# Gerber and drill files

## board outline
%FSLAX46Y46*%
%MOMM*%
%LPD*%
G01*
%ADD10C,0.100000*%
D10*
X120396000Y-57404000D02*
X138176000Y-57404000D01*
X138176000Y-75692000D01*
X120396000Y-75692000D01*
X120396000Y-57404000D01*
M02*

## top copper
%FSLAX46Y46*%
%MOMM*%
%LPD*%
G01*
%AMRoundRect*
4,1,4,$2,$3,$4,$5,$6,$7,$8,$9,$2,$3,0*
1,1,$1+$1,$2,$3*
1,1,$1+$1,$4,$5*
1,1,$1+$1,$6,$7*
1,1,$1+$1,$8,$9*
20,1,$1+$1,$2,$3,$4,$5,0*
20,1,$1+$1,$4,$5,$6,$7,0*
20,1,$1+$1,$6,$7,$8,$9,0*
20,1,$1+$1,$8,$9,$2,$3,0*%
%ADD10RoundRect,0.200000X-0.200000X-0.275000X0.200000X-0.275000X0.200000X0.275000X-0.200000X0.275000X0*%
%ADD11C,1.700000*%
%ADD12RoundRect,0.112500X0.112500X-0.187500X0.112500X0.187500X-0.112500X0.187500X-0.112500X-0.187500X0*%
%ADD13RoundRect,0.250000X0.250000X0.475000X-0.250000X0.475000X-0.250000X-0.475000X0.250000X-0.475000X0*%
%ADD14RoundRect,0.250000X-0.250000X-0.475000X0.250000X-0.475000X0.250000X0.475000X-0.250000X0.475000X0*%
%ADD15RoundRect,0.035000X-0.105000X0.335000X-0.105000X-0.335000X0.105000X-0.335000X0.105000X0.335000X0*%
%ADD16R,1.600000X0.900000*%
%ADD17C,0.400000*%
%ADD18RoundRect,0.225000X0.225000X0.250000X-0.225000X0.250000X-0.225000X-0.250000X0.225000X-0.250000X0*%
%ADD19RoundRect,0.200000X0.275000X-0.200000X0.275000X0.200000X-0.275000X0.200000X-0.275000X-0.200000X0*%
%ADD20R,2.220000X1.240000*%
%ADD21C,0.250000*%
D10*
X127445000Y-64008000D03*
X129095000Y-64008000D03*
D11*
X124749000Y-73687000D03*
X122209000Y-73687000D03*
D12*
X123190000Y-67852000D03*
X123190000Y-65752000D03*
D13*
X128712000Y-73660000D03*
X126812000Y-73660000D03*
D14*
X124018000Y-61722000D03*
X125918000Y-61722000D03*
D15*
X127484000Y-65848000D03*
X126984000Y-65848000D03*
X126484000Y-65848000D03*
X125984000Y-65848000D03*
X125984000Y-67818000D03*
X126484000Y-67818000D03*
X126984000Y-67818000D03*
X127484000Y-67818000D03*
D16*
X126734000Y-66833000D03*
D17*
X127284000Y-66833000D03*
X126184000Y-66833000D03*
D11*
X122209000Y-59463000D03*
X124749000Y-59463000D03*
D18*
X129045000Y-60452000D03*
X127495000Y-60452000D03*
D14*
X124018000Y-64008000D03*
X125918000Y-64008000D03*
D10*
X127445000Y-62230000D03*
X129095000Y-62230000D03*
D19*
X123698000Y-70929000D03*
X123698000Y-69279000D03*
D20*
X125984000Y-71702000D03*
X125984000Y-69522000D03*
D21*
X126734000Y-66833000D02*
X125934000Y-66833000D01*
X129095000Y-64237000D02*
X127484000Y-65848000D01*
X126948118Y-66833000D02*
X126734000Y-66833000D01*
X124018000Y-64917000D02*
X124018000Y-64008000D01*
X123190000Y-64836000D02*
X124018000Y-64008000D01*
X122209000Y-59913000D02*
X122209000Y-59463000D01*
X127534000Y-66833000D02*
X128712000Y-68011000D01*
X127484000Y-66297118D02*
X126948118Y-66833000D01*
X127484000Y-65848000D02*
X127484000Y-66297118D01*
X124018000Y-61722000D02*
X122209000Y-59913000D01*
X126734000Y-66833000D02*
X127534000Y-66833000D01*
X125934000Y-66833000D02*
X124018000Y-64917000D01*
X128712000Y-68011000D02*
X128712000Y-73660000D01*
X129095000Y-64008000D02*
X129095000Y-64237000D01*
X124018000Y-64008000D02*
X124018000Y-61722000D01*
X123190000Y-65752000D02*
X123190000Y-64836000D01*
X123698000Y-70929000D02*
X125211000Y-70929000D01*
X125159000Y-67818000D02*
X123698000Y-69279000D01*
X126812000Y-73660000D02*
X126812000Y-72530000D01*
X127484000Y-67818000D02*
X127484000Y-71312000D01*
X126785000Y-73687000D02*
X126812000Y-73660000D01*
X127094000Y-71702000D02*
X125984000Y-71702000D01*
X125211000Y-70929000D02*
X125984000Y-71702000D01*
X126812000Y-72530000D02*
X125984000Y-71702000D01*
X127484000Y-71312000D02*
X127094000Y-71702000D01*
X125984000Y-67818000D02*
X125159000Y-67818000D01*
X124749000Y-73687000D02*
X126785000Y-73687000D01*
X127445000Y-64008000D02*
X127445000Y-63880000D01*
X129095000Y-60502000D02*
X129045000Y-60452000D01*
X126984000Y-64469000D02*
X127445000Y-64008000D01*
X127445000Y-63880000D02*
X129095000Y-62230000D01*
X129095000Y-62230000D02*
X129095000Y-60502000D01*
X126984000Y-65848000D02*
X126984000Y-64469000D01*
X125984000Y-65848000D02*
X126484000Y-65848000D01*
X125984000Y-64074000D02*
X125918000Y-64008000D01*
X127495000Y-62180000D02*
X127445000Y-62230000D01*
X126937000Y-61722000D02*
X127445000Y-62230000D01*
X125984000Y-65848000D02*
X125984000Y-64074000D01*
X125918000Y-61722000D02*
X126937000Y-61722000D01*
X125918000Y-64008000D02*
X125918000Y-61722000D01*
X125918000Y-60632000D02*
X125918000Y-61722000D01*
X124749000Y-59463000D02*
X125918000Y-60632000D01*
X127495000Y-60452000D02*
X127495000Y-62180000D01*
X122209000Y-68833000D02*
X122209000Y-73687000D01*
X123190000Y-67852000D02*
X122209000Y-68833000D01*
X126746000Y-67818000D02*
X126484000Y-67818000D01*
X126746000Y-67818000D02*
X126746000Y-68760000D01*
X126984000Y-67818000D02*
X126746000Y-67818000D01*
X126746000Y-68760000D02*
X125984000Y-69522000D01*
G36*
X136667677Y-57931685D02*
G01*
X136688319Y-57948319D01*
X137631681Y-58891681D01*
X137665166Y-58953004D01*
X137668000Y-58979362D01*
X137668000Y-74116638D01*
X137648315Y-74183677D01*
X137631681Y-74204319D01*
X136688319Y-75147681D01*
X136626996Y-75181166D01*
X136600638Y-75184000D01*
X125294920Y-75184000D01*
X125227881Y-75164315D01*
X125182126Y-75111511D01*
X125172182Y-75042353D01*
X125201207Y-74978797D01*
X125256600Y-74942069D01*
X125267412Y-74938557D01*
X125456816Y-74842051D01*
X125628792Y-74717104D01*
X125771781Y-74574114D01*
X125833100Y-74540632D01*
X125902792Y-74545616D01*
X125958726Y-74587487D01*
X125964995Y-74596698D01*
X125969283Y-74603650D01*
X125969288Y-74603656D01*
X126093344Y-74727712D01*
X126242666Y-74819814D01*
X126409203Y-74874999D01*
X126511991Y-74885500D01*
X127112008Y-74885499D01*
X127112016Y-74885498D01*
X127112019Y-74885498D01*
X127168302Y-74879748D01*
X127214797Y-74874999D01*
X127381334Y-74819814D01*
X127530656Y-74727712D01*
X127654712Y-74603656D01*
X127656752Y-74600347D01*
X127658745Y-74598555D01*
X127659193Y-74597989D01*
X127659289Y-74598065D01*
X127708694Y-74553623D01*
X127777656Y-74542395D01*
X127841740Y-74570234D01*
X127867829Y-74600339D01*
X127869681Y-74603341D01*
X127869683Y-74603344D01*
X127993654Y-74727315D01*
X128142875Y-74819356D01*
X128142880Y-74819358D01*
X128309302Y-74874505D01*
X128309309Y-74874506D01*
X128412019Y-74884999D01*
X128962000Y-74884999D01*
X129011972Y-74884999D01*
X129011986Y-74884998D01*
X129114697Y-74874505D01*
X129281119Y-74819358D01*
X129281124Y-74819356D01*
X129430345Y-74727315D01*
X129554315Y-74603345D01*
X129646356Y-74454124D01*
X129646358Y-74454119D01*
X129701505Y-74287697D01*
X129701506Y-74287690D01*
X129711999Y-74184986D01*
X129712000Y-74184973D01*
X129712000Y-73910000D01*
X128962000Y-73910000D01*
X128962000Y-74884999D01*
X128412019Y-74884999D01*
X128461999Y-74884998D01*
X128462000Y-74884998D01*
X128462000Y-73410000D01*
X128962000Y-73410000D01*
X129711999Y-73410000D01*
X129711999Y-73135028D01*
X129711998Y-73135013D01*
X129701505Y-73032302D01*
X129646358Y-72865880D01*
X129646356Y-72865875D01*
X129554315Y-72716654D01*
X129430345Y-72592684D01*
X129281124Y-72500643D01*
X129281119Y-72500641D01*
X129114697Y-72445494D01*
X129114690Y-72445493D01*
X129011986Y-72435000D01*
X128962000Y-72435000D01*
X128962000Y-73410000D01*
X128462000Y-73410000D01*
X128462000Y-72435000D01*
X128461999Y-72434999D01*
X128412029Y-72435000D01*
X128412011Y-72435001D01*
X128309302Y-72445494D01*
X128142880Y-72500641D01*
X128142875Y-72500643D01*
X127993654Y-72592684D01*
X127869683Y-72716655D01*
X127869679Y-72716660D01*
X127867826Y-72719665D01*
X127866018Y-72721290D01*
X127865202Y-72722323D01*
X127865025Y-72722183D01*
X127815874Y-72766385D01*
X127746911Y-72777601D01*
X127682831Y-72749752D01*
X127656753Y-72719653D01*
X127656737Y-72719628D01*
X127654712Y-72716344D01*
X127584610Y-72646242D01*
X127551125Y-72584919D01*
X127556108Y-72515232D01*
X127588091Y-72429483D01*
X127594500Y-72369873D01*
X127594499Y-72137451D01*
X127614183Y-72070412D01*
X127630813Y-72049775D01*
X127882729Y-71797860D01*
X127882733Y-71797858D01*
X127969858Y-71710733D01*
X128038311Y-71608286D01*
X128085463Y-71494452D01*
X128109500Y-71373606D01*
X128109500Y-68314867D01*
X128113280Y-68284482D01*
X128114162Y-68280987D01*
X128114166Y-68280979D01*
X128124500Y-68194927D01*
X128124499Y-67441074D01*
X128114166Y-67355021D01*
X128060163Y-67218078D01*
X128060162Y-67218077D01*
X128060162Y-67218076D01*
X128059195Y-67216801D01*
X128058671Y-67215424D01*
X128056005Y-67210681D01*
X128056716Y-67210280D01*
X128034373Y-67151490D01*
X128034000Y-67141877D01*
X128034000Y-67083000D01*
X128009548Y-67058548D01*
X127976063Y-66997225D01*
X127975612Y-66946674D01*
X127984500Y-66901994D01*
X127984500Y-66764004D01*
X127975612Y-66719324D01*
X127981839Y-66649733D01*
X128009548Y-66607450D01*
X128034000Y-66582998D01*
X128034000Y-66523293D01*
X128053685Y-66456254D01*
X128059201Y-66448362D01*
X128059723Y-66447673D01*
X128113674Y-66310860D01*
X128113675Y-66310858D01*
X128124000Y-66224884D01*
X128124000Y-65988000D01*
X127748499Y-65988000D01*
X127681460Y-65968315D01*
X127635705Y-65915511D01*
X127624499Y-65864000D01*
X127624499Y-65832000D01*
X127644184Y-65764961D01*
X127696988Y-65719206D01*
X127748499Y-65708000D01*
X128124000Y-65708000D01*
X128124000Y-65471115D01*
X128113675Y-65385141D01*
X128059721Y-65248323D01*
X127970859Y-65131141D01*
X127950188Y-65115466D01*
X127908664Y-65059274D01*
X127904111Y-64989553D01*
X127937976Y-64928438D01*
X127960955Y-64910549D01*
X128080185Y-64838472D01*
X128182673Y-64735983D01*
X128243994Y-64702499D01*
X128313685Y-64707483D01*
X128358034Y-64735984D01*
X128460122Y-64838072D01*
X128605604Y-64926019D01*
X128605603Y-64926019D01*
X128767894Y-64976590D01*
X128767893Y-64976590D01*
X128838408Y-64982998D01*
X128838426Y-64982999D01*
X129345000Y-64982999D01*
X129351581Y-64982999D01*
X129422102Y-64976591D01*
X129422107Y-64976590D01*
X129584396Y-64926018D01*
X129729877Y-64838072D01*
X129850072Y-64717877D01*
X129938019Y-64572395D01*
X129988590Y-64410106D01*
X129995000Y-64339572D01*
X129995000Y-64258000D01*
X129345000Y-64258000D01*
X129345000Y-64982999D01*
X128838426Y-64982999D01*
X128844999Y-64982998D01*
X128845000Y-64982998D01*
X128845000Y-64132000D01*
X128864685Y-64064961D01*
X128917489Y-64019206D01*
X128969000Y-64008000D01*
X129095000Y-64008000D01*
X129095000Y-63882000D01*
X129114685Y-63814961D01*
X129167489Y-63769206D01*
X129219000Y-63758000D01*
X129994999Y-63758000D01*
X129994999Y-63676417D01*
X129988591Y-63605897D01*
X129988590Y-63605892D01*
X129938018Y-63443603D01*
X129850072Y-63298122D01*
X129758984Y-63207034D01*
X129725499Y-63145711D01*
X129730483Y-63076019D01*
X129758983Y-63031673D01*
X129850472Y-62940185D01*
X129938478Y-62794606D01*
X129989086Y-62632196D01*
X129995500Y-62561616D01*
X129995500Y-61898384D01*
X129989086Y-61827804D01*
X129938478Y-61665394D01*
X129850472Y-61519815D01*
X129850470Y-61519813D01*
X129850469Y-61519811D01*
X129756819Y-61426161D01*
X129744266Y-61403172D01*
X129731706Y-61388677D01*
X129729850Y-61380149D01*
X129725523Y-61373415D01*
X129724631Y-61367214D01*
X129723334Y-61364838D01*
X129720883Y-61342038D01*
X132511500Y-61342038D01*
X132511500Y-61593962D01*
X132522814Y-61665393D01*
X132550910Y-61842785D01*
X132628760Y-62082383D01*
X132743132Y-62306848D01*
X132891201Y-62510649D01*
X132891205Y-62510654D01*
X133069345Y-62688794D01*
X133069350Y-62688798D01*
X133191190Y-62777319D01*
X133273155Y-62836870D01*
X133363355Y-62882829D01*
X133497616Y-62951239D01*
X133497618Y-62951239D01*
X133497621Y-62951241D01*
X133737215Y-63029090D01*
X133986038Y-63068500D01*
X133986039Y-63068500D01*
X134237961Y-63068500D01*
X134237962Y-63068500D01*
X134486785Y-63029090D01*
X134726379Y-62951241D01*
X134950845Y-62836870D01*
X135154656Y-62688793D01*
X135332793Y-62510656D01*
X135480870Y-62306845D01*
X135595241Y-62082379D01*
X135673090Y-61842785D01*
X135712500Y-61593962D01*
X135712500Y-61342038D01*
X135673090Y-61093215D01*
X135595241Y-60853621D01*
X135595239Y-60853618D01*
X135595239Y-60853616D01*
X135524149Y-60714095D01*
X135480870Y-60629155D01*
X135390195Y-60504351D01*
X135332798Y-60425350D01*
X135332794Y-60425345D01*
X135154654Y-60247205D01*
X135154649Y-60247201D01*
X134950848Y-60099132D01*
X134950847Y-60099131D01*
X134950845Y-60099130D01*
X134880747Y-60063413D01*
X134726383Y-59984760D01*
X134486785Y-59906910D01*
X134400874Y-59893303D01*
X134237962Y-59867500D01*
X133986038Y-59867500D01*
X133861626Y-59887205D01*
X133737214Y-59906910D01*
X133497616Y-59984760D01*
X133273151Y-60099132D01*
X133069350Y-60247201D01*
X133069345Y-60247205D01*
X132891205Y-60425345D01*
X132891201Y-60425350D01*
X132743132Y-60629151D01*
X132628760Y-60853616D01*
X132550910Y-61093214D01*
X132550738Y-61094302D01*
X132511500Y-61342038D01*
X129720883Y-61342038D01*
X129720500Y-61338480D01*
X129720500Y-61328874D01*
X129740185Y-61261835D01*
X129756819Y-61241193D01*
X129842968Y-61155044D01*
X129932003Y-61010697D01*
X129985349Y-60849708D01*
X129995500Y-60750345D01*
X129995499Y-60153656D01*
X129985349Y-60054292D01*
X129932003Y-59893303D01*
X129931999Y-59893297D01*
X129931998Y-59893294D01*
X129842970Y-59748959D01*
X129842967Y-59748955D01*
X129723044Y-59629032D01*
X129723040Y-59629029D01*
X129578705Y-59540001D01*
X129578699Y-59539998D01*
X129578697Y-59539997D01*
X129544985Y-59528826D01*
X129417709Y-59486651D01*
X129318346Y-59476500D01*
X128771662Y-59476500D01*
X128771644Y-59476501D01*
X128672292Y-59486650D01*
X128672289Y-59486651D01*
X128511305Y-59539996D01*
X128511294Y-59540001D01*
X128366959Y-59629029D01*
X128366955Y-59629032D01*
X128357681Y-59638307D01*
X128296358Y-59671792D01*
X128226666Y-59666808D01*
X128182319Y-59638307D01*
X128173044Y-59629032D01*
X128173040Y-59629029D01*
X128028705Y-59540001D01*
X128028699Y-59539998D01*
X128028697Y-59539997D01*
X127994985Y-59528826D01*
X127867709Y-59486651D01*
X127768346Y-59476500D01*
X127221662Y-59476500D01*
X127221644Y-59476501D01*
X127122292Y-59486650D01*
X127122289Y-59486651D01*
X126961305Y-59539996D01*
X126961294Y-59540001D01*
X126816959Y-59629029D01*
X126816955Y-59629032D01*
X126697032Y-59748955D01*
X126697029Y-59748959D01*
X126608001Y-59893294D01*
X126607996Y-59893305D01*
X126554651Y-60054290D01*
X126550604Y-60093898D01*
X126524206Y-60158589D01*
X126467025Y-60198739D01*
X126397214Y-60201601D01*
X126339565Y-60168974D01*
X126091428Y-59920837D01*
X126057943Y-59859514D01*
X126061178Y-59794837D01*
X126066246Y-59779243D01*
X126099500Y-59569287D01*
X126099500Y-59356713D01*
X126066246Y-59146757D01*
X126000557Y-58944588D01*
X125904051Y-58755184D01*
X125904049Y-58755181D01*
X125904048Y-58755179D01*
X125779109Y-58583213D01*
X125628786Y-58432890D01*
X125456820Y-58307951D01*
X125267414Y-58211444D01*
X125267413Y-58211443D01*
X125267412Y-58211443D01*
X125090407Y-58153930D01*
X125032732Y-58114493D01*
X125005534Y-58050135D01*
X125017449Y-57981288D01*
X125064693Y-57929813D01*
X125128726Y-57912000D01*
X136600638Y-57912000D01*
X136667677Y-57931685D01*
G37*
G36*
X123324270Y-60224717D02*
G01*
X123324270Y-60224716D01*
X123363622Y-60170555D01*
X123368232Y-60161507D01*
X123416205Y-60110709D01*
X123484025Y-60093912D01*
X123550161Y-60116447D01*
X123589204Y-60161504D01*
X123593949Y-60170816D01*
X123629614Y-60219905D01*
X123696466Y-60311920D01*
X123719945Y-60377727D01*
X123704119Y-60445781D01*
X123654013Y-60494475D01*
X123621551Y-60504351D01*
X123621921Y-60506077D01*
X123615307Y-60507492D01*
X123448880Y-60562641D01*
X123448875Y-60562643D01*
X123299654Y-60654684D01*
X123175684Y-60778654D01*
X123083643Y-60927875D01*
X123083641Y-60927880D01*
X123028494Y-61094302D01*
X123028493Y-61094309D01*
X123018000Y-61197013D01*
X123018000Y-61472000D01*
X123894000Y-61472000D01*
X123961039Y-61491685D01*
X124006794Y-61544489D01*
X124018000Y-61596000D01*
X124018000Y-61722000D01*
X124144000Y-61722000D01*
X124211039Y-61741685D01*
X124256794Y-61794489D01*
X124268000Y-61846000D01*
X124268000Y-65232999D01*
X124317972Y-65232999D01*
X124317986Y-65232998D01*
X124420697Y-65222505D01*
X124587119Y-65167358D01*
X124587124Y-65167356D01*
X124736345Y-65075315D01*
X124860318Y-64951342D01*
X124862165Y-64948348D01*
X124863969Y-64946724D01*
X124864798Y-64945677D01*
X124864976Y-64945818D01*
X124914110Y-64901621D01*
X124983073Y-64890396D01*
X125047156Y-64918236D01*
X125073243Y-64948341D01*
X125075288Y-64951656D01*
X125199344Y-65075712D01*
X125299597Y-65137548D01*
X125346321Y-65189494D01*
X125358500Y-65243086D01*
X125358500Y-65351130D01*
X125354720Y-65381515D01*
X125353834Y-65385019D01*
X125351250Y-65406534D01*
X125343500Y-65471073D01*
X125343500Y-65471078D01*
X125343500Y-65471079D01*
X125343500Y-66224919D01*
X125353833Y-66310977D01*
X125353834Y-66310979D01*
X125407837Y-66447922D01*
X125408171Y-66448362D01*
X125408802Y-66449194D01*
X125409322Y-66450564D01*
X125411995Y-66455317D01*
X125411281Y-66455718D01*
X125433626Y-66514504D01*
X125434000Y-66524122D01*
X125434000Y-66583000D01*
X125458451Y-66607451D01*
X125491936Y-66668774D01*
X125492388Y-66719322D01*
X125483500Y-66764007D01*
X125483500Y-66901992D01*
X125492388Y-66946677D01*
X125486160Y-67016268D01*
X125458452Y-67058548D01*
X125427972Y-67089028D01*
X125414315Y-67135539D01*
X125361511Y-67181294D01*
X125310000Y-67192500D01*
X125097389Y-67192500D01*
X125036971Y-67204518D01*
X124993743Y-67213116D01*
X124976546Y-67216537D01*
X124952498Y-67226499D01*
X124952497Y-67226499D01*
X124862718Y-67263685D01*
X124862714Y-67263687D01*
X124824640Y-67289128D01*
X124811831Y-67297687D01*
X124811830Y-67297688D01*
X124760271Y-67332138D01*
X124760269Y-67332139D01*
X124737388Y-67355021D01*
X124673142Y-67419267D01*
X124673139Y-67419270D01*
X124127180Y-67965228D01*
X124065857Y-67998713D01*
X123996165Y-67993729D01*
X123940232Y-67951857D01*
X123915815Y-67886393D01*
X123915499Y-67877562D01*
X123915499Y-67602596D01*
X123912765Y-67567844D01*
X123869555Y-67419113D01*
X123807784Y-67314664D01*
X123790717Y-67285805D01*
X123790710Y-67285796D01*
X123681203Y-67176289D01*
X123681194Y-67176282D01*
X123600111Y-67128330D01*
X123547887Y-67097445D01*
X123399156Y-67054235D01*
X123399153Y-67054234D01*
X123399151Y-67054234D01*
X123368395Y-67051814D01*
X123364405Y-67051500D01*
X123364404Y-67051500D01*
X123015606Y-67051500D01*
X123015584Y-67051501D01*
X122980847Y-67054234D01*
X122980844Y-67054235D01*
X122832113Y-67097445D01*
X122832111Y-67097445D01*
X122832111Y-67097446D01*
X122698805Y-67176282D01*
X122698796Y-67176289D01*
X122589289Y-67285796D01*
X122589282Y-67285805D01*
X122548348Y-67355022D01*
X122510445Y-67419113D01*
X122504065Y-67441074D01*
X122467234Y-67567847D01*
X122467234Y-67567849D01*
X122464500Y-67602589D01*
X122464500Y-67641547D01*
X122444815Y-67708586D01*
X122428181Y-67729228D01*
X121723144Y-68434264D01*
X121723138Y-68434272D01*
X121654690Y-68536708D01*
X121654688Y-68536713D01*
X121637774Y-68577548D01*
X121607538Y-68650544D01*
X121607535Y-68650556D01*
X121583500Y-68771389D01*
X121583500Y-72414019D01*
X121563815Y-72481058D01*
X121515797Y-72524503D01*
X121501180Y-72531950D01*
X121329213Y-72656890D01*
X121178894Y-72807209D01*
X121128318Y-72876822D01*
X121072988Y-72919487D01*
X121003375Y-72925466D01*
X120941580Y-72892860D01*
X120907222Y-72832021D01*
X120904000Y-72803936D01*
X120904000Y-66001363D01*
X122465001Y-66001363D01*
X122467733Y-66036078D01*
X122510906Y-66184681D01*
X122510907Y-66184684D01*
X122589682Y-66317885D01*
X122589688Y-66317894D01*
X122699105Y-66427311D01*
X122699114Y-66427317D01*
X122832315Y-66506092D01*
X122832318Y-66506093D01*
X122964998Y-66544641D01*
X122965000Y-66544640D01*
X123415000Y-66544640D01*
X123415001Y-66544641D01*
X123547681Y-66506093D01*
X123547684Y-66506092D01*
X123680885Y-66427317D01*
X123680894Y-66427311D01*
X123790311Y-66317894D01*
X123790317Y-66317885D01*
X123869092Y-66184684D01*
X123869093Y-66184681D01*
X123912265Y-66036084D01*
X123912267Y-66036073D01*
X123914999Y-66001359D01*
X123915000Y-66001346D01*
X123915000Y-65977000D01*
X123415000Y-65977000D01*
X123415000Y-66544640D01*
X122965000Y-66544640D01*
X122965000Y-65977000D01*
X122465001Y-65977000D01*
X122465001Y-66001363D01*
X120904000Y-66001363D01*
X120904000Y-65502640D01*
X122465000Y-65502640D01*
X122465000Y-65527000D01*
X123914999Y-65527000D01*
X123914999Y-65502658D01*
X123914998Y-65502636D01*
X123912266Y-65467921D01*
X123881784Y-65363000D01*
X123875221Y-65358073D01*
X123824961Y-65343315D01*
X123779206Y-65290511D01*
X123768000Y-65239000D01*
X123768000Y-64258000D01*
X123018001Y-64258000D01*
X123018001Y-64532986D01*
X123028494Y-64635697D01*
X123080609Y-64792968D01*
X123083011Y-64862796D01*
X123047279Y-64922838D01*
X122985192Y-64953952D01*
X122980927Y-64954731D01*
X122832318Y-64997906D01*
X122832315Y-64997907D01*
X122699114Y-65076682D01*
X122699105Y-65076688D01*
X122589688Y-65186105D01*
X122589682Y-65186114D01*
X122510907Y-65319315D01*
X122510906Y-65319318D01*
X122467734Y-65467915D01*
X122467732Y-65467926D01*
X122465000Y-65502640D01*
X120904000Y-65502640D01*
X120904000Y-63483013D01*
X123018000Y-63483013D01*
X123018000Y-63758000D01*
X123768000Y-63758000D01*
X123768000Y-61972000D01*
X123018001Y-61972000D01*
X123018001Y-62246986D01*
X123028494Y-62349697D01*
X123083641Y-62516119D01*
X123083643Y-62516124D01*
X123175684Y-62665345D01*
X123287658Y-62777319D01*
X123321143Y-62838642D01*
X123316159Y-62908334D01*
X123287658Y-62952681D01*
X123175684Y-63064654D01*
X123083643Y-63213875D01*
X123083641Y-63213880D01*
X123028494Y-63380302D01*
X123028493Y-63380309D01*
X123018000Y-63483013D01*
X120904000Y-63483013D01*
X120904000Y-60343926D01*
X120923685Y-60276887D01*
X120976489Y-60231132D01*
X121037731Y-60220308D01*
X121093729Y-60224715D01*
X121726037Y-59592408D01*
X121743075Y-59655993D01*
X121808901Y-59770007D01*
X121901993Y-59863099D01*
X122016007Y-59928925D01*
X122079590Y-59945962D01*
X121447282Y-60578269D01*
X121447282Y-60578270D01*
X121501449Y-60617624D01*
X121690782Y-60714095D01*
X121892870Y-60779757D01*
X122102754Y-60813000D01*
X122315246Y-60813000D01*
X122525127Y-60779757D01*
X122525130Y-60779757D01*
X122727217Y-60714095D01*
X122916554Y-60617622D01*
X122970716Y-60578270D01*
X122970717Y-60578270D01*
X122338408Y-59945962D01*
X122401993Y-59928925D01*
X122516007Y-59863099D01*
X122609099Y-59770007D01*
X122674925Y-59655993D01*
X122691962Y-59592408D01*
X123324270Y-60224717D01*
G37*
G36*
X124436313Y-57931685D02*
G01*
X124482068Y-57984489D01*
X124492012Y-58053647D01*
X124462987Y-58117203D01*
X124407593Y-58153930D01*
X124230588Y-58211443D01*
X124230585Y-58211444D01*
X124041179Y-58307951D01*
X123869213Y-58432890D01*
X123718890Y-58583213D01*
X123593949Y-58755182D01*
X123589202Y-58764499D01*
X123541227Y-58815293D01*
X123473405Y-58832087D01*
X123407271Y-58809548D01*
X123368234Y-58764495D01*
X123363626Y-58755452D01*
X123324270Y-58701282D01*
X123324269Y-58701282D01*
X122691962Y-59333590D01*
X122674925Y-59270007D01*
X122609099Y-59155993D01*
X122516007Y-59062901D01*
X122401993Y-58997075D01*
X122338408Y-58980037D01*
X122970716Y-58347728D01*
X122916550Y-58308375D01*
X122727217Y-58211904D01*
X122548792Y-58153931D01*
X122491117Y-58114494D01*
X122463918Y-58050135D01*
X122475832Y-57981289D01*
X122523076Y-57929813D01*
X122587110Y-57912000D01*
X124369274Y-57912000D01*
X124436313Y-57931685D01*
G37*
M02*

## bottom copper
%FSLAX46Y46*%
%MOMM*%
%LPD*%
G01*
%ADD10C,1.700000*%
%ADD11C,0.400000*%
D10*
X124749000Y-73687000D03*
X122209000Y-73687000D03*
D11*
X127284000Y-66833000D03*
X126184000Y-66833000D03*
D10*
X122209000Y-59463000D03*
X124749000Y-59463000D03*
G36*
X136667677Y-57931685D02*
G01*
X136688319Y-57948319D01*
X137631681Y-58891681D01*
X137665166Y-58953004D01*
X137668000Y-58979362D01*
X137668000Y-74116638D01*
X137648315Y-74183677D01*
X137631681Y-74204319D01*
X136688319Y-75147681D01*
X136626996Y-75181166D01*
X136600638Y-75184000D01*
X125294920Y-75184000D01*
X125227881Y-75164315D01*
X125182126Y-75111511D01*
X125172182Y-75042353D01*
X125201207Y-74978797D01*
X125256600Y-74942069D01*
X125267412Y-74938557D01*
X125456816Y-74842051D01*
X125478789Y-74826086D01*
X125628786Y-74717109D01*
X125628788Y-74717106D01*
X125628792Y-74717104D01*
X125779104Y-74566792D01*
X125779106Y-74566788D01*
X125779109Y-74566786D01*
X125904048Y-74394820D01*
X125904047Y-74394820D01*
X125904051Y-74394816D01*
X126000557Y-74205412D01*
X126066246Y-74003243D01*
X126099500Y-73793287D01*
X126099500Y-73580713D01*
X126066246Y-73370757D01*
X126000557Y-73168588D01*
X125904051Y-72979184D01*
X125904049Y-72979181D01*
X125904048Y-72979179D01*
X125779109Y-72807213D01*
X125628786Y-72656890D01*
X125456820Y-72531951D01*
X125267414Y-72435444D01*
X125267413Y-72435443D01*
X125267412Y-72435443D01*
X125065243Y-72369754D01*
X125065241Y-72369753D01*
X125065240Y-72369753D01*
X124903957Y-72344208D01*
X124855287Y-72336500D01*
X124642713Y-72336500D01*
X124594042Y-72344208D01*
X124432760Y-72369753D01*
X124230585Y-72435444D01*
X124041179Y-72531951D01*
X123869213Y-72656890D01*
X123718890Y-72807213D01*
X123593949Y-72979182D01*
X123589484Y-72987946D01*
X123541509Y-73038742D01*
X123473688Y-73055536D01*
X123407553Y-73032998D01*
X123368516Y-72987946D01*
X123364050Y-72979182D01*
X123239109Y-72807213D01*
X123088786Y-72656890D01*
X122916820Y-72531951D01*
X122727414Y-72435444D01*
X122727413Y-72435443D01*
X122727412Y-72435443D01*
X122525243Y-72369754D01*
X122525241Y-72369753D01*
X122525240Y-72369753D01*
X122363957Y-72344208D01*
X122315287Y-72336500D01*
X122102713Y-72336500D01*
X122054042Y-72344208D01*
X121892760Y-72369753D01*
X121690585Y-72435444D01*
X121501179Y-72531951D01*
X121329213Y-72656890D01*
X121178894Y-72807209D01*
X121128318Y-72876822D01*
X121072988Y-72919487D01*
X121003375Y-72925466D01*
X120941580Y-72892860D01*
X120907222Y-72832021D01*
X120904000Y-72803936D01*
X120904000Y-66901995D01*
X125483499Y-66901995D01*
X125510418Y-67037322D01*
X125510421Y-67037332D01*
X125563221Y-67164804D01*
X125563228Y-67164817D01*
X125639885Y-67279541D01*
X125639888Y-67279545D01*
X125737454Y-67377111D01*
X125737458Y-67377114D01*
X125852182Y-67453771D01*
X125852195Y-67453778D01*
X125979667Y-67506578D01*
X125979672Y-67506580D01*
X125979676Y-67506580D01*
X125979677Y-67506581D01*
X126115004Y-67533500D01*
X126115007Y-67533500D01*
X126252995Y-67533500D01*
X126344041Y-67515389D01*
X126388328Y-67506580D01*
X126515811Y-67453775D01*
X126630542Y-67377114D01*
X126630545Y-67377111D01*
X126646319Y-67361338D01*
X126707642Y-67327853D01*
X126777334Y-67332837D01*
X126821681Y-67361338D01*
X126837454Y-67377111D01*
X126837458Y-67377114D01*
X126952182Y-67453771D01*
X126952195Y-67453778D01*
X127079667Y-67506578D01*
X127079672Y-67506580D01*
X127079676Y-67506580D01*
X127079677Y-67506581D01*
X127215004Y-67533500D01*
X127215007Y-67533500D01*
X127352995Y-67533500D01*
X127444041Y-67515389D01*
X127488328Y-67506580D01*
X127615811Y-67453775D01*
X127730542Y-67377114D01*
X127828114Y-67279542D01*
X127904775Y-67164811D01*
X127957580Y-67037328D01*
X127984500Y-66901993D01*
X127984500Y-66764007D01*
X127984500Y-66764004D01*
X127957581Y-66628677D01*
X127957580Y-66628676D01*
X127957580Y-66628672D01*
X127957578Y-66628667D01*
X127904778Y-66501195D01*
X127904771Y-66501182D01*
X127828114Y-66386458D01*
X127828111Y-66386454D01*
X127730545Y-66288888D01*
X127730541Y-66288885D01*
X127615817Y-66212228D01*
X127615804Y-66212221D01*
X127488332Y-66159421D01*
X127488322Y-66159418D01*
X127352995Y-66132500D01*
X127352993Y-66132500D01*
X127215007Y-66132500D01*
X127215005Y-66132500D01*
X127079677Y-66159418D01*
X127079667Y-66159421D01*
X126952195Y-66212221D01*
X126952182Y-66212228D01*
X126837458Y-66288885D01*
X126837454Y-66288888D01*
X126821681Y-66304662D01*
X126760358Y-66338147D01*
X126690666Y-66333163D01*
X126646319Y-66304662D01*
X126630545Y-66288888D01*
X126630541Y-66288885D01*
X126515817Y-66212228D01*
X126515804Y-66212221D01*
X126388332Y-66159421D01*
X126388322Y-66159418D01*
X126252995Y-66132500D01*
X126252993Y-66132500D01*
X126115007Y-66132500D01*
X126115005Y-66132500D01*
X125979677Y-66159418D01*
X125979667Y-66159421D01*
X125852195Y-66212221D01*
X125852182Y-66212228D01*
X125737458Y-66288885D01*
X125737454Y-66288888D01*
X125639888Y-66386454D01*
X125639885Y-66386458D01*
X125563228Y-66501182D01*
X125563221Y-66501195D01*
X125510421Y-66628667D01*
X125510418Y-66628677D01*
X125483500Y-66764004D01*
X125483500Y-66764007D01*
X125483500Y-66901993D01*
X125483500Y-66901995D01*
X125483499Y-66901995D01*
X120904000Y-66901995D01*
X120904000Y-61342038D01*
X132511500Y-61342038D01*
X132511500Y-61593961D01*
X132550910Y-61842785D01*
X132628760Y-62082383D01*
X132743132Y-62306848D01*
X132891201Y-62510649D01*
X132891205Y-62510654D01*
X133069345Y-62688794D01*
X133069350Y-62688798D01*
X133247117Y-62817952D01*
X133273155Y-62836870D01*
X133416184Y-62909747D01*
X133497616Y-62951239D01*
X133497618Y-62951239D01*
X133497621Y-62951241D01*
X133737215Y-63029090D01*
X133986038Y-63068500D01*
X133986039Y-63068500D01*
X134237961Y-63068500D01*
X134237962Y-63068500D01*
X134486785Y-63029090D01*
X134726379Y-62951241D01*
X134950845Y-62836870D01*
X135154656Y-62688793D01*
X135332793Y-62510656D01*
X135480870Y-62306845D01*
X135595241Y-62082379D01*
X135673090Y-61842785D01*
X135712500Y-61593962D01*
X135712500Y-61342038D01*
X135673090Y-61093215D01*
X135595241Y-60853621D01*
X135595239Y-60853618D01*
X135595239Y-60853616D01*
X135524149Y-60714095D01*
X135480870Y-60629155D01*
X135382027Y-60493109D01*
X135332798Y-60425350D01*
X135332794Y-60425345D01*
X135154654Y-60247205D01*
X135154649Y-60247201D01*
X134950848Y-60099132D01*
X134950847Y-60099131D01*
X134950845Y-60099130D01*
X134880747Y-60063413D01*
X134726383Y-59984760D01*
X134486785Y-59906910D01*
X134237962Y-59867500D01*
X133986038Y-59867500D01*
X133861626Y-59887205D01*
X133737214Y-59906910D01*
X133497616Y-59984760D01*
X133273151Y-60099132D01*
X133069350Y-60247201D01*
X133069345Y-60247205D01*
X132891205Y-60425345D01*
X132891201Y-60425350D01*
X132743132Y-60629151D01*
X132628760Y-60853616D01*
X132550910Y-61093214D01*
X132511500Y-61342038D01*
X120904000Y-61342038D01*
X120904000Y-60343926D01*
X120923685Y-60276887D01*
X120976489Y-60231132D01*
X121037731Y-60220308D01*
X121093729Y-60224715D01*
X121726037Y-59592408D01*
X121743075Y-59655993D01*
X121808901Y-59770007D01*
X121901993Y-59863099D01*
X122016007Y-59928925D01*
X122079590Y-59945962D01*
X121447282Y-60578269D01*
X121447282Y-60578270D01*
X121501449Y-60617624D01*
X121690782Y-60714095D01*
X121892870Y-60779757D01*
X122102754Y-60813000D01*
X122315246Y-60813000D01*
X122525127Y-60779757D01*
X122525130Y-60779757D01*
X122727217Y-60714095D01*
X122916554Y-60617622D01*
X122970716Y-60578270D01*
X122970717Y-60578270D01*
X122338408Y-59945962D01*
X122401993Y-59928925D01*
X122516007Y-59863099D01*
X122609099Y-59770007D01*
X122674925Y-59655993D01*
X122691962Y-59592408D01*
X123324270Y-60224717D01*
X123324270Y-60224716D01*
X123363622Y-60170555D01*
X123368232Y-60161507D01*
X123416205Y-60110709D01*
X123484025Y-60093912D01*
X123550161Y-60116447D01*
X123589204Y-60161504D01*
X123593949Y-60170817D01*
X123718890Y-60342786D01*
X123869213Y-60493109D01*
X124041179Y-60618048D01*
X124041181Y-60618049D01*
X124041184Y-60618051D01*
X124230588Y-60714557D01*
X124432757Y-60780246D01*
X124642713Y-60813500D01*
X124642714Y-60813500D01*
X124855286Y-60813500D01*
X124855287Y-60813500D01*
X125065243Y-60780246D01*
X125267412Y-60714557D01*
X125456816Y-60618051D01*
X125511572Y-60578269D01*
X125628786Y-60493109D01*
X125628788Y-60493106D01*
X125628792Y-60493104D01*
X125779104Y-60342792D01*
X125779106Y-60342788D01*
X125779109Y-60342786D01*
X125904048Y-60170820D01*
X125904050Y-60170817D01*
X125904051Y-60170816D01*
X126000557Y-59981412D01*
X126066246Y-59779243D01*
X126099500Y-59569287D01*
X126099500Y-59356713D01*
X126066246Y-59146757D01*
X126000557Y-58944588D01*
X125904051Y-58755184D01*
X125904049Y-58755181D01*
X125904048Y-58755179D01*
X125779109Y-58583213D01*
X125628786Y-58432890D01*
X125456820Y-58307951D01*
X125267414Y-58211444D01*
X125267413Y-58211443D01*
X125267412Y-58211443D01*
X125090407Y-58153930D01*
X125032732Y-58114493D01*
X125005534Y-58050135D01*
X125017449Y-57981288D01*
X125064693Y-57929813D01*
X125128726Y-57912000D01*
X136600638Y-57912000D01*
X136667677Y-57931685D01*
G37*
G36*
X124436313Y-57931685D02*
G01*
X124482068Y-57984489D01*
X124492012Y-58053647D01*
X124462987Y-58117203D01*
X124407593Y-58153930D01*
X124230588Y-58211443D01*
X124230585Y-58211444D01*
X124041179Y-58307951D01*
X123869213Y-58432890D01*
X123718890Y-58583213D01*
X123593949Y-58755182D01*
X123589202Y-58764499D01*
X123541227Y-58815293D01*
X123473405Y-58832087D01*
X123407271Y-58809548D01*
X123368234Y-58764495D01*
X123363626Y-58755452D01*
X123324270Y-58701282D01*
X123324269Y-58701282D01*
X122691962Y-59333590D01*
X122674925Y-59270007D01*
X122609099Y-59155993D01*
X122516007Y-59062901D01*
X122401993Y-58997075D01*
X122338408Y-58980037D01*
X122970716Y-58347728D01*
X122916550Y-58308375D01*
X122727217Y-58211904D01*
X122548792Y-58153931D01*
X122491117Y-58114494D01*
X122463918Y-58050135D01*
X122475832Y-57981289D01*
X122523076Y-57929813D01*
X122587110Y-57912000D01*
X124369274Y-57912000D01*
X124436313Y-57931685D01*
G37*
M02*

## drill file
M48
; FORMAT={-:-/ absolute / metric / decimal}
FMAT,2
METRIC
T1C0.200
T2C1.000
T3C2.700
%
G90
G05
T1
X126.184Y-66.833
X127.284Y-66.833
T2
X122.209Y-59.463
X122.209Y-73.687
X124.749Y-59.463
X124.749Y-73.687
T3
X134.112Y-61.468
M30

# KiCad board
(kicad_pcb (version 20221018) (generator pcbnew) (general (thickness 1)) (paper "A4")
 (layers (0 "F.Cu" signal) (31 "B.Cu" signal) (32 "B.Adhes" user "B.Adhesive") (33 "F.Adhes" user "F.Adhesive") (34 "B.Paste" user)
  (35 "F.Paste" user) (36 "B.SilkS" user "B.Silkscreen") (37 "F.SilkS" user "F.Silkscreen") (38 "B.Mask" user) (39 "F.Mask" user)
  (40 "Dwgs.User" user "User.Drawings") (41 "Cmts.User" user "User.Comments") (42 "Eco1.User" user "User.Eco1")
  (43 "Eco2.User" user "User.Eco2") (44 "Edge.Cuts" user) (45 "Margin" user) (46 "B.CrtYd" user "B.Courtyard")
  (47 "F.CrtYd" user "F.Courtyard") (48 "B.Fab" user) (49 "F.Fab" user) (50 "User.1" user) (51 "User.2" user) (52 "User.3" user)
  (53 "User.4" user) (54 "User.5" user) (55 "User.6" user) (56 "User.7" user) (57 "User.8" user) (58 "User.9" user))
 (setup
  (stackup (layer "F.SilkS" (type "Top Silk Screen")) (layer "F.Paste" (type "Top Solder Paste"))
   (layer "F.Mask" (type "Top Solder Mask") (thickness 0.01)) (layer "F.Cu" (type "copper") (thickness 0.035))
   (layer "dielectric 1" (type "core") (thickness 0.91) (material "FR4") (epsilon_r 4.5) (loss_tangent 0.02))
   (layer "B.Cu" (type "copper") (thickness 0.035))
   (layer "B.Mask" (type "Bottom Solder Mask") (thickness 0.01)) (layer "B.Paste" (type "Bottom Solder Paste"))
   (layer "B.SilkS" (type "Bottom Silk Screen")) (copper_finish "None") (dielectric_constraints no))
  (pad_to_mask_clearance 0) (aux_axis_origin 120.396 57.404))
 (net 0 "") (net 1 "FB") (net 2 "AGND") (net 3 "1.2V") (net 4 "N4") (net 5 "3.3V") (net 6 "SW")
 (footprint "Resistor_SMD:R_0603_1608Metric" (layer "F.Cu") (at 128.27 64.008)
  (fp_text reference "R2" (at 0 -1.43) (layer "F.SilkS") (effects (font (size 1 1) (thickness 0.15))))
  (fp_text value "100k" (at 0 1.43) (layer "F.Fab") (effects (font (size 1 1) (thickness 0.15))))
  (pad "1" smd roundrect (at -0.825 0) (size 0.8 0.95) (layers "F.Cu" "F.Paste" "F.Mask") (roundrect_rratio 0.25) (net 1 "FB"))
  (pad "2" smd roundrect (at 0.825 0) (size 0.8 0.95) (layers "F.Cu" "F.Paste" "F.Mask") (roundrect_rratio 0.25) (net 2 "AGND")))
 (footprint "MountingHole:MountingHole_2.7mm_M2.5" (layer "F.Cu") (at 134.112 61.468)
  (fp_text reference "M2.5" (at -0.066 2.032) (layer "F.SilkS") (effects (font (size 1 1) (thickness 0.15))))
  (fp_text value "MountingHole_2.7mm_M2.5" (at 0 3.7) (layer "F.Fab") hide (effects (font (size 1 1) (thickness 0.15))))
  (pad "" np_thru_hole circle (at 0 0) (size 2.7 2.7) (drill 2.7) (layers "F&B.Cu" "*.Mask")))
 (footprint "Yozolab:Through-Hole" (layer "F.Cu") (at 124.749 73.687 180)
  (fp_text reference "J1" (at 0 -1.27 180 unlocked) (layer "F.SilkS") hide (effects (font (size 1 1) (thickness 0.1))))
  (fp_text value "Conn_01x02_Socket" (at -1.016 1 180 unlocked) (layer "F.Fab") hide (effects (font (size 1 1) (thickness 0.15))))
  (pad "1" thru_hole circle (at 0 0 180) (size 1.7 1.7) (drill oval 1) (layers "*.Cu" "*.Mask") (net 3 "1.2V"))
  (pad "2" thru_hole circle (at 2.54 0 180) (size 1.7 1.7) (drill oval 1) (layers "*.Cu" "*.Mask") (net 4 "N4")))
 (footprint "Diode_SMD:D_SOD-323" (layer "F.Cu") (at 123.19 66.802 90)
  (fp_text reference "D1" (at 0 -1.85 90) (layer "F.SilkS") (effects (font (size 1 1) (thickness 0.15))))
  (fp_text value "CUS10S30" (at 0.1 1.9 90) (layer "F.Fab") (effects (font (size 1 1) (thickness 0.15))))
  (pad "1" smd roundrect (at -1.05 0 90) (size 0.6 0.45) (layers "F.Cu" "F.Paste" "F.Mask") (roundrect_rratio 0.25) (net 4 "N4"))
  (pad "2" smd roundrect (at 1.05 0 90) (size 0.6 0.45) (layers "F.Cu" "F.Paste" "F.Mask") (roundrect_rratio 0.25) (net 2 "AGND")))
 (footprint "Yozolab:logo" (layer "F.Cu") (at 136.144 70.612 90)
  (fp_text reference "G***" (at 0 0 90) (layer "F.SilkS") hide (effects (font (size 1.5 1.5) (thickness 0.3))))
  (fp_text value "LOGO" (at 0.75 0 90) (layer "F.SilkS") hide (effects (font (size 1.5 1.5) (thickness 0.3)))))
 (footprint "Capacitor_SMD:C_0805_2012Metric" (layer "F.Cu") (at 127.762 73.66 180)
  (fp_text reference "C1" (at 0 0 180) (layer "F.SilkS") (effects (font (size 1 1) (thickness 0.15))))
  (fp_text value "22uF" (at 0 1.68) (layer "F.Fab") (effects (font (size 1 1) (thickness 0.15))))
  (pad "1" smd roundrect (at -0.95 0 180) (size 1 1.45) (layers "F.Cu" "F.Paste" "F.Mask") (roundrect_rratio 0.25) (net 2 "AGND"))
  (pad "2" smd roundrect (at 0.95 0 180) (size 1 1.45) (layers "F.Cu" "F.Paste" "F.Mask") (roundrect_rratio 0.25) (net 3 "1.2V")))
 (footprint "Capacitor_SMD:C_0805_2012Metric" (layer "F.Cu") (at 124.968 61.722)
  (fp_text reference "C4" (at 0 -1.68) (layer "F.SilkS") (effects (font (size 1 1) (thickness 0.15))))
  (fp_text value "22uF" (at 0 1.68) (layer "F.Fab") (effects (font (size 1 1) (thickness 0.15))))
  (pad "1" smd roundrect (at -0.95 0) (size 1 1.45) (layers "F.Cu" "F.Paste" "F.Mask") (roundrect_rratio 0.25) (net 2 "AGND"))
  (pad "2" smd roundrect (at 0.95 0) (size 1 1.45) (layers "F.Cu" "F.Paste" "F.Mask") (roundrect_rratio 0.25) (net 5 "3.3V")))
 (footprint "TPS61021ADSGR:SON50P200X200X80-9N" (layer "F.Cu") (at 126.734 66.833 -90)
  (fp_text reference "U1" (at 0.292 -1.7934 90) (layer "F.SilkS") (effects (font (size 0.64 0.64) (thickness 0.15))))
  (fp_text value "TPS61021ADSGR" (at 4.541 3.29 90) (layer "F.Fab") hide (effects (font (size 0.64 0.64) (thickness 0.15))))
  (pad "1" smd roundrect (at -0.985 -0.75 270) (size 0.74 0.28) (layers "F.Cu" "F.Paste" "F.Mask") (roundrect_rratio 0.125) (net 2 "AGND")
   (solder_mask_margin 0.102))
  (pad "2" smd roundrect (at -0.985 -0.25 270) (size 0.74 0.28) (layers "F.Cu" "F.Paste" "F.Mask") (roundrect_rratio 0.125) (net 1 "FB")
   (solder_mask_margin 0.102))
  (pad "3" smd roundrect (at -0.985 0.25 270) (size 0.74 0.28) (layers "F.Cu" "F.Paste" "F.Mask") (roundrect_rratio 0.125) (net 5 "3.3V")
   (solder_mask_margin 0.102))
  (pad "4" smd roundrect (at -0.985 0.75 270) (size 0.74 0.28) (layers "F.Cu" "F.Paste" "F.Mask") (roundrect_rratio 0.125) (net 5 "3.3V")
   (solder_mask_margin 0.102))
  (pad "5" smd roundrect (at 0.985 0.75 270) (size 0.74 0.28) (layers "F.Cu" "F.Paste" "F.Mask") (roundrect_rratio 0.125) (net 3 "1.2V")
   (solder_mask_margin 0.102))
  (pad "6" smd roundrect (at 0.985 0.25 270) (size 0.74 0.28) (layers "F.Cu" "F.Paste" "F.Mask") (roundrect_rratio 0.125) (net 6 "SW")
   (solder_mask_margin 0.102))
  (pad "7" smd roundrect (at 0.985 -0.25 270) (size 0.74 0.28) (layers "F.Cu" "F.Paste" "F.Mask") (roundrect_rratio 0.125) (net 6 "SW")
   (solder_mask_margin 0.102))
  (pad "8" smd roundrect (at 0.985 -0.75 270) (size 0.74 0.28) (layers "F.Cu" "F.Paste" "F.Mask") (roundrect_rratio 0.125) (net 3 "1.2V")
   (solder_mask_margin 0.102))
  (pad "9" smd rect (at 0 0 270) (size 0.9 1.6) (layers "F.Cu" "F.Mask") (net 2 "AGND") (solder_mask_margin 0.102))
  (pad "9_1" thru_hole circle (at 0 -0.55 270) (size 0.4 0.4) (drill 0.2) (layers "*.Cu"))
  (pad "9_2" thru_hole circle (at 0 0.55 270) (size 0.4 0.4) (drill 0.2) (layers "*.Cu")))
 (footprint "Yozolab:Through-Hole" (layer "F.Cu") (at 122.209 59.463)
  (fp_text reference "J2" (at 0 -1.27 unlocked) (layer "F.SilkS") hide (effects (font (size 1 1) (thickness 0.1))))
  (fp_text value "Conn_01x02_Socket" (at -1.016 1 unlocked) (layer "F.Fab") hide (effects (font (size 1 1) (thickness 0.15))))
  (pad "1" thru_hole circle (at 0 0) (size 1.7 1.7) (drill oval 1) (layers "*.Cu" "*.Mask") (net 2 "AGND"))
  (pad "2" thru_hole circle (at 2.54 0) (size 1.7 1.7) (drill oval 1) (layers "*.Cu" "*.Mask") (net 5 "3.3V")))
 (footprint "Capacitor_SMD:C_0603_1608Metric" (layer "F.Cu") (at 128.27 60.452 180)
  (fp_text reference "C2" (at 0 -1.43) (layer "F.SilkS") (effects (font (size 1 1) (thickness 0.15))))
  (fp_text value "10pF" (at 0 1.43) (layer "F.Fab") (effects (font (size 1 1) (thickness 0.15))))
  (pad "1" smd roundrect (at -0.775 0 180) (size 0.9 0.95) (layers "F.Cu" "F.Paste" "F.Mask") (roundrect_rratio 0.25) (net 1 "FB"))
  (pad "2" smd roundrect (at 0.775 0 180) (size 0.9 0.95) (layers "F.Cu" "F.Paste" "F.Mask") (roundrect_rratio 0.25) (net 5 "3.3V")))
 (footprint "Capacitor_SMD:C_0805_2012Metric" (layer "F.Cu") (at 124.968 64.008)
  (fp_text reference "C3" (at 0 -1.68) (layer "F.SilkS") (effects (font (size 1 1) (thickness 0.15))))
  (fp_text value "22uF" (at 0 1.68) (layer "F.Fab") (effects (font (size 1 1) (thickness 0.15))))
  (pad "1" smd roundrect (at -0.95 0) (size 1 1.45) (layers "F.Cu" "F.Paste" "F.Mask") (roundrect_rratio 0.25) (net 2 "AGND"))
  (pad "2" smd roundrect (at 0.95 0) (size 1 1.45) (layers "F.Cu" "F.Paste" "F.Mask") (roundrect_rratio 0.25) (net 5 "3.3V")))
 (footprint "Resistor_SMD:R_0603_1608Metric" (layer "F.Cu") (at 128.27 62.23)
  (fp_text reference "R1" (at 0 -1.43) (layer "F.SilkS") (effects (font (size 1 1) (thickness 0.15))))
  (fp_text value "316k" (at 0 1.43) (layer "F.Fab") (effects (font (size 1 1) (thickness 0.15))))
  (pad "1" smd roundrect (at -0.825 0) (size 0.8 0.95) (layers "F.Cu" "F.Paste" "F.Mask") (roundrect_rratio 0.25) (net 5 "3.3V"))
  (pad "2" smd roundrect (at 0.825 0) (size 0.8 0.95) (layers "F.Cu" "F.Paste" "F.Mask") (roundrect_rratio 0.25) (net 1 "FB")))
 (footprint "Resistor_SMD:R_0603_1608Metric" (layer "F.Cu") (at 123.698 70.104 90)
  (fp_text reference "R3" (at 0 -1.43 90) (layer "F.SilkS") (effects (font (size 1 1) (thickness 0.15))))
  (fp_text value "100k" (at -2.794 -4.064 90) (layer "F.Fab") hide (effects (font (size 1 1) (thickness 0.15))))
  (pad "1" smd roundrect (at -0.825 0 90) (size 0.8 0.95) (layers "F.Cu" "F.Paste" "F.Mask") (roundrect_rratio 0.25) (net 3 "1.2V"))
  (pad "2" smd roundrect (at 0.825 0 90) (size 0.8 0.95) (layers "F.Cu" "F.Paste" "F.Mask") (roundrect_rratio 0.25) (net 3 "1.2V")))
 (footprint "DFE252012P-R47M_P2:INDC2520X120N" (layer "F.Cu") (at 125.984 70.612 90)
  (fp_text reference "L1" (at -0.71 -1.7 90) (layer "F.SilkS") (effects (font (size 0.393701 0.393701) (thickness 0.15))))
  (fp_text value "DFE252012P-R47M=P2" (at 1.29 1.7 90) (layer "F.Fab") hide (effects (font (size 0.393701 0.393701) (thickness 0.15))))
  (pad "1" smd rect (at -1.09 0 90) (size 1.24 2.22) (layers "F.Cu" "F.Paste" "F.Mask") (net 3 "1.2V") (solder_mask_margin 0.102))
  (pad "2" smd rect (at 1.09 0 90) (size 1.24 2.22) (layers "F.Cu" "F.Paste" "F.Mask") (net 6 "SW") (solder_mask_margin 0.102)))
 (gr_rect (start 120.396 57.404) (end 138.176 75.692) (stroke (width 0.1) (type default)) (fill none) (layer "Edge.Cuts"))
 (segment (start 126.734 66.833) (end 125.934 66.833) (width 0.25) (layer "F.Cu") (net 2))
 (segment (start 129.095 64.237) (end 127.484 65.848) (width 0.25) (layer "F.Cu") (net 2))
 (segment (start 126.948118 66.833) (end 126.734 66.833) (width 0.25) (layer "F.Cu") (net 2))
 (segment (start 124.018 64.917) (end 124.018 64.008) (width 0.25) (layer "F.Cu") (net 2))
 (segment (start 123.19 64.836) (end 124.018 64.008) (width 0.25) (layer "F.Cu") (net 2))
 (segment (start 122.209 59.913) (end 122.209 59.463) (width 0.25) (layer "F.Cu") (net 2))
 (segment (start 127.534 66.833) (end 128.712 68.011) (width 0.25) (layer "F.Cu") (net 2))
 (segment (start 127.484 66.297118) (end 126.948118 66.833) (width 0.25) (layer "F.Cu") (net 2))
 (segment (start 127.484 65.848) (end 127.484 66.297118) (width 0.25) (layer "F.Cu") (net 2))
 (segment (start 124.018 61.722) (end 122.209 59.913) (width 0.25) (layer "F.Cu") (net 2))
 (segment (start 126.734 66.833) (end 127.534 66.833) (width 0.25) (layer "F.Cu") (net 2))
 (segment (start 125.934 66.833) (end 124.018 64.917) (width 0.25) (layer "F.Cu") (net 2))
 (segment (start 128.712 68.011) (end 128.712 73.66) (width 0.25) (layer "F.Cu") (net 2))
 (segment (start 129.095 64.008) (end 129.095 64.237) (width 0.25) (layer "F.Cu") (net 2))
 (segment (start 124.018 64.008) (end 124.018 61.722) (width 0.25) (layer "F.Cu") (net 2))
 (segment (start 123.19 65.752) (end 123.19 64.836) (width 0.25) (layer "F.Cu") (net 2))
 (segment (start 123.698 70.929) (end 125.211 70.929) (width 0.25) (layer "F.Cu") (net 3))
 (segment (start 125.159 67.818) (end 123.698 69.279) (width 0.25) (layer "F.Cu") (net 3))
 (segment (start 126.812 73.66) (end 126.812 72.53) (width 0.25) (layer "F.Cu") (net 3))
 (segment (start 127.484 67.818) (end 127.484 71.312) (width 0.25) (layer "F.Cu") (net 3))
 (segment (start 126.785 73.687) (end 126.812 73.66) (width 0.25) (layer "F.Cu") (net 3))
 (segment (start 127.094 71.702) (end 125.984 71.702) (width 0.25) (layer "F.Cu") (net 3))
 (segment (start 125.211 70.929) (end 125.984 71.702) (width 0.25) (layer "F.Cu") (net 3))
 (segment (start 126.812 72.53) (end 125.984 71.702) (width 0.25) (layer "F.Cu") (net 3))
 (segment (start 127.484 71.312) (end 127.094 71.702) (width 0.25) (layer "F.Cu") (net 3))
 (segment (start 125.984 67.818) (end 125.159 67.818) (width 0.25) (layer "F.Cu") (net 3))
 (segment (start 124.749 73.687) (end 126.785 73.687) (width 0.25) (layer "F.Cu") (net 3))
 (segment (start 127.445 64.008) (end 127.445 63.88) (width 0.25) (layer "F.Cu") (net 1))
 (segment (start 129.095 60.502) (end 129.045 60.452) (width 0.25) (layer "F.Cu") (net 1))
 (segment (start 126.984 64.469) (end 127.445 64.008) (width 0.25) (layer "F.Cu") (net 1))
 (segment (start 127.445 63.88) (end 129.095 62.23) (width 0.25) (layer "F.Cu") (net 1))
 (segment (start 129.095 62.23) (end 129.095 60.502) (width 0.25) (layer "F.Cu") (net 1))
 (segment (start 126.984 65.848) (end 126.984 64.469) (width 0.25) (layer "F.Cu") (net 1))
 (segment (start 125.984 65.848) (end 126.484 65.848) (width 0.25) (layer "F.Cu") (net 5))
 (segment (start 125.984 64.074) (end 125.918 64.008) (width 0.25) (layer "F.Cu") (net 5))
 (segment (start 127.495 62.18) (end 127.445 62.23) (width 0.25) (layer "F.Cu") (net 5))
 (segment (start 126.937 61.722) (end 127.445 62.23) (width 0.25) (layer "F.Cu") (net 5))
 (segment (start 125.984 65.848) (end 125.984 64.074) (width 0.25) (layer "F.Cu") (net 5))
 (segment (start 125.918 61.722) (end 126.937 61.722) (width 0.25) (layer "F.Cu") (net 5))
 (segment (start 125.918 64.008) (end 125.918 61.722) (width 0.25) (layer "F.Cu") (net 5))
 (segment (start 125.918 60.632) (end 125.918 61.722) (width 0.25) (layer "F.Cu") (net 5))
 (segment (start 124.749 59.463) (end 125.918 60.632) (width 0.25) (layer "F.Cu") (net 5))
 (segment (start 127.495 60.452) (end 127.495 62.18) (width 0.25) (layer "F.Cu") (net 5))
 (segment (start 122.209 68.833) (end 122.209 73.687) (width 0.25) (layer "F.Cu") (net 4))
 (segment (start 123.19 67.852) (end 122.209 68.833) (width 0.25) (layer "F.Cu") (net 4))
 (segment (start 126.746 67.818) (end 126.484 67.818) (width 0.25) (layer "F.Cu") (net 6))
 (segment (start 126.746 67.818) (end 126.746 68.76) (width 0.25) (layer "F.Cu") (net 6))
 (segment (start 126.984 67.818) (end 126.746 67.818) (width 0.25) (layer "F.Cu") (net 6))
 (segment (start 126.746 68.76) (end 125.984 69.522) (width 0.25) (layer "F.Cu") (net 6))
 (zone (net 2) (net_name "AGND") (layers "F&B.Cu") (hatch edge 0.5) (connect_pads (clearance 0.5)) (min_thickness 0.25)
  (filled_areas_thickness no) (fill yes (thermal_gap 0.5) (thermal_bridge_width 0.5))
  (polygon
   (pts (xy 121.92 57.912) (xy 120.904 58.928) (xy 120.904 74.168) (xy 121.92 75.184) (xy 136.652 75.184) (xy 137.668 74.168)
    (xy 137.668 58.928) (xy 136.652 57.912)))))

